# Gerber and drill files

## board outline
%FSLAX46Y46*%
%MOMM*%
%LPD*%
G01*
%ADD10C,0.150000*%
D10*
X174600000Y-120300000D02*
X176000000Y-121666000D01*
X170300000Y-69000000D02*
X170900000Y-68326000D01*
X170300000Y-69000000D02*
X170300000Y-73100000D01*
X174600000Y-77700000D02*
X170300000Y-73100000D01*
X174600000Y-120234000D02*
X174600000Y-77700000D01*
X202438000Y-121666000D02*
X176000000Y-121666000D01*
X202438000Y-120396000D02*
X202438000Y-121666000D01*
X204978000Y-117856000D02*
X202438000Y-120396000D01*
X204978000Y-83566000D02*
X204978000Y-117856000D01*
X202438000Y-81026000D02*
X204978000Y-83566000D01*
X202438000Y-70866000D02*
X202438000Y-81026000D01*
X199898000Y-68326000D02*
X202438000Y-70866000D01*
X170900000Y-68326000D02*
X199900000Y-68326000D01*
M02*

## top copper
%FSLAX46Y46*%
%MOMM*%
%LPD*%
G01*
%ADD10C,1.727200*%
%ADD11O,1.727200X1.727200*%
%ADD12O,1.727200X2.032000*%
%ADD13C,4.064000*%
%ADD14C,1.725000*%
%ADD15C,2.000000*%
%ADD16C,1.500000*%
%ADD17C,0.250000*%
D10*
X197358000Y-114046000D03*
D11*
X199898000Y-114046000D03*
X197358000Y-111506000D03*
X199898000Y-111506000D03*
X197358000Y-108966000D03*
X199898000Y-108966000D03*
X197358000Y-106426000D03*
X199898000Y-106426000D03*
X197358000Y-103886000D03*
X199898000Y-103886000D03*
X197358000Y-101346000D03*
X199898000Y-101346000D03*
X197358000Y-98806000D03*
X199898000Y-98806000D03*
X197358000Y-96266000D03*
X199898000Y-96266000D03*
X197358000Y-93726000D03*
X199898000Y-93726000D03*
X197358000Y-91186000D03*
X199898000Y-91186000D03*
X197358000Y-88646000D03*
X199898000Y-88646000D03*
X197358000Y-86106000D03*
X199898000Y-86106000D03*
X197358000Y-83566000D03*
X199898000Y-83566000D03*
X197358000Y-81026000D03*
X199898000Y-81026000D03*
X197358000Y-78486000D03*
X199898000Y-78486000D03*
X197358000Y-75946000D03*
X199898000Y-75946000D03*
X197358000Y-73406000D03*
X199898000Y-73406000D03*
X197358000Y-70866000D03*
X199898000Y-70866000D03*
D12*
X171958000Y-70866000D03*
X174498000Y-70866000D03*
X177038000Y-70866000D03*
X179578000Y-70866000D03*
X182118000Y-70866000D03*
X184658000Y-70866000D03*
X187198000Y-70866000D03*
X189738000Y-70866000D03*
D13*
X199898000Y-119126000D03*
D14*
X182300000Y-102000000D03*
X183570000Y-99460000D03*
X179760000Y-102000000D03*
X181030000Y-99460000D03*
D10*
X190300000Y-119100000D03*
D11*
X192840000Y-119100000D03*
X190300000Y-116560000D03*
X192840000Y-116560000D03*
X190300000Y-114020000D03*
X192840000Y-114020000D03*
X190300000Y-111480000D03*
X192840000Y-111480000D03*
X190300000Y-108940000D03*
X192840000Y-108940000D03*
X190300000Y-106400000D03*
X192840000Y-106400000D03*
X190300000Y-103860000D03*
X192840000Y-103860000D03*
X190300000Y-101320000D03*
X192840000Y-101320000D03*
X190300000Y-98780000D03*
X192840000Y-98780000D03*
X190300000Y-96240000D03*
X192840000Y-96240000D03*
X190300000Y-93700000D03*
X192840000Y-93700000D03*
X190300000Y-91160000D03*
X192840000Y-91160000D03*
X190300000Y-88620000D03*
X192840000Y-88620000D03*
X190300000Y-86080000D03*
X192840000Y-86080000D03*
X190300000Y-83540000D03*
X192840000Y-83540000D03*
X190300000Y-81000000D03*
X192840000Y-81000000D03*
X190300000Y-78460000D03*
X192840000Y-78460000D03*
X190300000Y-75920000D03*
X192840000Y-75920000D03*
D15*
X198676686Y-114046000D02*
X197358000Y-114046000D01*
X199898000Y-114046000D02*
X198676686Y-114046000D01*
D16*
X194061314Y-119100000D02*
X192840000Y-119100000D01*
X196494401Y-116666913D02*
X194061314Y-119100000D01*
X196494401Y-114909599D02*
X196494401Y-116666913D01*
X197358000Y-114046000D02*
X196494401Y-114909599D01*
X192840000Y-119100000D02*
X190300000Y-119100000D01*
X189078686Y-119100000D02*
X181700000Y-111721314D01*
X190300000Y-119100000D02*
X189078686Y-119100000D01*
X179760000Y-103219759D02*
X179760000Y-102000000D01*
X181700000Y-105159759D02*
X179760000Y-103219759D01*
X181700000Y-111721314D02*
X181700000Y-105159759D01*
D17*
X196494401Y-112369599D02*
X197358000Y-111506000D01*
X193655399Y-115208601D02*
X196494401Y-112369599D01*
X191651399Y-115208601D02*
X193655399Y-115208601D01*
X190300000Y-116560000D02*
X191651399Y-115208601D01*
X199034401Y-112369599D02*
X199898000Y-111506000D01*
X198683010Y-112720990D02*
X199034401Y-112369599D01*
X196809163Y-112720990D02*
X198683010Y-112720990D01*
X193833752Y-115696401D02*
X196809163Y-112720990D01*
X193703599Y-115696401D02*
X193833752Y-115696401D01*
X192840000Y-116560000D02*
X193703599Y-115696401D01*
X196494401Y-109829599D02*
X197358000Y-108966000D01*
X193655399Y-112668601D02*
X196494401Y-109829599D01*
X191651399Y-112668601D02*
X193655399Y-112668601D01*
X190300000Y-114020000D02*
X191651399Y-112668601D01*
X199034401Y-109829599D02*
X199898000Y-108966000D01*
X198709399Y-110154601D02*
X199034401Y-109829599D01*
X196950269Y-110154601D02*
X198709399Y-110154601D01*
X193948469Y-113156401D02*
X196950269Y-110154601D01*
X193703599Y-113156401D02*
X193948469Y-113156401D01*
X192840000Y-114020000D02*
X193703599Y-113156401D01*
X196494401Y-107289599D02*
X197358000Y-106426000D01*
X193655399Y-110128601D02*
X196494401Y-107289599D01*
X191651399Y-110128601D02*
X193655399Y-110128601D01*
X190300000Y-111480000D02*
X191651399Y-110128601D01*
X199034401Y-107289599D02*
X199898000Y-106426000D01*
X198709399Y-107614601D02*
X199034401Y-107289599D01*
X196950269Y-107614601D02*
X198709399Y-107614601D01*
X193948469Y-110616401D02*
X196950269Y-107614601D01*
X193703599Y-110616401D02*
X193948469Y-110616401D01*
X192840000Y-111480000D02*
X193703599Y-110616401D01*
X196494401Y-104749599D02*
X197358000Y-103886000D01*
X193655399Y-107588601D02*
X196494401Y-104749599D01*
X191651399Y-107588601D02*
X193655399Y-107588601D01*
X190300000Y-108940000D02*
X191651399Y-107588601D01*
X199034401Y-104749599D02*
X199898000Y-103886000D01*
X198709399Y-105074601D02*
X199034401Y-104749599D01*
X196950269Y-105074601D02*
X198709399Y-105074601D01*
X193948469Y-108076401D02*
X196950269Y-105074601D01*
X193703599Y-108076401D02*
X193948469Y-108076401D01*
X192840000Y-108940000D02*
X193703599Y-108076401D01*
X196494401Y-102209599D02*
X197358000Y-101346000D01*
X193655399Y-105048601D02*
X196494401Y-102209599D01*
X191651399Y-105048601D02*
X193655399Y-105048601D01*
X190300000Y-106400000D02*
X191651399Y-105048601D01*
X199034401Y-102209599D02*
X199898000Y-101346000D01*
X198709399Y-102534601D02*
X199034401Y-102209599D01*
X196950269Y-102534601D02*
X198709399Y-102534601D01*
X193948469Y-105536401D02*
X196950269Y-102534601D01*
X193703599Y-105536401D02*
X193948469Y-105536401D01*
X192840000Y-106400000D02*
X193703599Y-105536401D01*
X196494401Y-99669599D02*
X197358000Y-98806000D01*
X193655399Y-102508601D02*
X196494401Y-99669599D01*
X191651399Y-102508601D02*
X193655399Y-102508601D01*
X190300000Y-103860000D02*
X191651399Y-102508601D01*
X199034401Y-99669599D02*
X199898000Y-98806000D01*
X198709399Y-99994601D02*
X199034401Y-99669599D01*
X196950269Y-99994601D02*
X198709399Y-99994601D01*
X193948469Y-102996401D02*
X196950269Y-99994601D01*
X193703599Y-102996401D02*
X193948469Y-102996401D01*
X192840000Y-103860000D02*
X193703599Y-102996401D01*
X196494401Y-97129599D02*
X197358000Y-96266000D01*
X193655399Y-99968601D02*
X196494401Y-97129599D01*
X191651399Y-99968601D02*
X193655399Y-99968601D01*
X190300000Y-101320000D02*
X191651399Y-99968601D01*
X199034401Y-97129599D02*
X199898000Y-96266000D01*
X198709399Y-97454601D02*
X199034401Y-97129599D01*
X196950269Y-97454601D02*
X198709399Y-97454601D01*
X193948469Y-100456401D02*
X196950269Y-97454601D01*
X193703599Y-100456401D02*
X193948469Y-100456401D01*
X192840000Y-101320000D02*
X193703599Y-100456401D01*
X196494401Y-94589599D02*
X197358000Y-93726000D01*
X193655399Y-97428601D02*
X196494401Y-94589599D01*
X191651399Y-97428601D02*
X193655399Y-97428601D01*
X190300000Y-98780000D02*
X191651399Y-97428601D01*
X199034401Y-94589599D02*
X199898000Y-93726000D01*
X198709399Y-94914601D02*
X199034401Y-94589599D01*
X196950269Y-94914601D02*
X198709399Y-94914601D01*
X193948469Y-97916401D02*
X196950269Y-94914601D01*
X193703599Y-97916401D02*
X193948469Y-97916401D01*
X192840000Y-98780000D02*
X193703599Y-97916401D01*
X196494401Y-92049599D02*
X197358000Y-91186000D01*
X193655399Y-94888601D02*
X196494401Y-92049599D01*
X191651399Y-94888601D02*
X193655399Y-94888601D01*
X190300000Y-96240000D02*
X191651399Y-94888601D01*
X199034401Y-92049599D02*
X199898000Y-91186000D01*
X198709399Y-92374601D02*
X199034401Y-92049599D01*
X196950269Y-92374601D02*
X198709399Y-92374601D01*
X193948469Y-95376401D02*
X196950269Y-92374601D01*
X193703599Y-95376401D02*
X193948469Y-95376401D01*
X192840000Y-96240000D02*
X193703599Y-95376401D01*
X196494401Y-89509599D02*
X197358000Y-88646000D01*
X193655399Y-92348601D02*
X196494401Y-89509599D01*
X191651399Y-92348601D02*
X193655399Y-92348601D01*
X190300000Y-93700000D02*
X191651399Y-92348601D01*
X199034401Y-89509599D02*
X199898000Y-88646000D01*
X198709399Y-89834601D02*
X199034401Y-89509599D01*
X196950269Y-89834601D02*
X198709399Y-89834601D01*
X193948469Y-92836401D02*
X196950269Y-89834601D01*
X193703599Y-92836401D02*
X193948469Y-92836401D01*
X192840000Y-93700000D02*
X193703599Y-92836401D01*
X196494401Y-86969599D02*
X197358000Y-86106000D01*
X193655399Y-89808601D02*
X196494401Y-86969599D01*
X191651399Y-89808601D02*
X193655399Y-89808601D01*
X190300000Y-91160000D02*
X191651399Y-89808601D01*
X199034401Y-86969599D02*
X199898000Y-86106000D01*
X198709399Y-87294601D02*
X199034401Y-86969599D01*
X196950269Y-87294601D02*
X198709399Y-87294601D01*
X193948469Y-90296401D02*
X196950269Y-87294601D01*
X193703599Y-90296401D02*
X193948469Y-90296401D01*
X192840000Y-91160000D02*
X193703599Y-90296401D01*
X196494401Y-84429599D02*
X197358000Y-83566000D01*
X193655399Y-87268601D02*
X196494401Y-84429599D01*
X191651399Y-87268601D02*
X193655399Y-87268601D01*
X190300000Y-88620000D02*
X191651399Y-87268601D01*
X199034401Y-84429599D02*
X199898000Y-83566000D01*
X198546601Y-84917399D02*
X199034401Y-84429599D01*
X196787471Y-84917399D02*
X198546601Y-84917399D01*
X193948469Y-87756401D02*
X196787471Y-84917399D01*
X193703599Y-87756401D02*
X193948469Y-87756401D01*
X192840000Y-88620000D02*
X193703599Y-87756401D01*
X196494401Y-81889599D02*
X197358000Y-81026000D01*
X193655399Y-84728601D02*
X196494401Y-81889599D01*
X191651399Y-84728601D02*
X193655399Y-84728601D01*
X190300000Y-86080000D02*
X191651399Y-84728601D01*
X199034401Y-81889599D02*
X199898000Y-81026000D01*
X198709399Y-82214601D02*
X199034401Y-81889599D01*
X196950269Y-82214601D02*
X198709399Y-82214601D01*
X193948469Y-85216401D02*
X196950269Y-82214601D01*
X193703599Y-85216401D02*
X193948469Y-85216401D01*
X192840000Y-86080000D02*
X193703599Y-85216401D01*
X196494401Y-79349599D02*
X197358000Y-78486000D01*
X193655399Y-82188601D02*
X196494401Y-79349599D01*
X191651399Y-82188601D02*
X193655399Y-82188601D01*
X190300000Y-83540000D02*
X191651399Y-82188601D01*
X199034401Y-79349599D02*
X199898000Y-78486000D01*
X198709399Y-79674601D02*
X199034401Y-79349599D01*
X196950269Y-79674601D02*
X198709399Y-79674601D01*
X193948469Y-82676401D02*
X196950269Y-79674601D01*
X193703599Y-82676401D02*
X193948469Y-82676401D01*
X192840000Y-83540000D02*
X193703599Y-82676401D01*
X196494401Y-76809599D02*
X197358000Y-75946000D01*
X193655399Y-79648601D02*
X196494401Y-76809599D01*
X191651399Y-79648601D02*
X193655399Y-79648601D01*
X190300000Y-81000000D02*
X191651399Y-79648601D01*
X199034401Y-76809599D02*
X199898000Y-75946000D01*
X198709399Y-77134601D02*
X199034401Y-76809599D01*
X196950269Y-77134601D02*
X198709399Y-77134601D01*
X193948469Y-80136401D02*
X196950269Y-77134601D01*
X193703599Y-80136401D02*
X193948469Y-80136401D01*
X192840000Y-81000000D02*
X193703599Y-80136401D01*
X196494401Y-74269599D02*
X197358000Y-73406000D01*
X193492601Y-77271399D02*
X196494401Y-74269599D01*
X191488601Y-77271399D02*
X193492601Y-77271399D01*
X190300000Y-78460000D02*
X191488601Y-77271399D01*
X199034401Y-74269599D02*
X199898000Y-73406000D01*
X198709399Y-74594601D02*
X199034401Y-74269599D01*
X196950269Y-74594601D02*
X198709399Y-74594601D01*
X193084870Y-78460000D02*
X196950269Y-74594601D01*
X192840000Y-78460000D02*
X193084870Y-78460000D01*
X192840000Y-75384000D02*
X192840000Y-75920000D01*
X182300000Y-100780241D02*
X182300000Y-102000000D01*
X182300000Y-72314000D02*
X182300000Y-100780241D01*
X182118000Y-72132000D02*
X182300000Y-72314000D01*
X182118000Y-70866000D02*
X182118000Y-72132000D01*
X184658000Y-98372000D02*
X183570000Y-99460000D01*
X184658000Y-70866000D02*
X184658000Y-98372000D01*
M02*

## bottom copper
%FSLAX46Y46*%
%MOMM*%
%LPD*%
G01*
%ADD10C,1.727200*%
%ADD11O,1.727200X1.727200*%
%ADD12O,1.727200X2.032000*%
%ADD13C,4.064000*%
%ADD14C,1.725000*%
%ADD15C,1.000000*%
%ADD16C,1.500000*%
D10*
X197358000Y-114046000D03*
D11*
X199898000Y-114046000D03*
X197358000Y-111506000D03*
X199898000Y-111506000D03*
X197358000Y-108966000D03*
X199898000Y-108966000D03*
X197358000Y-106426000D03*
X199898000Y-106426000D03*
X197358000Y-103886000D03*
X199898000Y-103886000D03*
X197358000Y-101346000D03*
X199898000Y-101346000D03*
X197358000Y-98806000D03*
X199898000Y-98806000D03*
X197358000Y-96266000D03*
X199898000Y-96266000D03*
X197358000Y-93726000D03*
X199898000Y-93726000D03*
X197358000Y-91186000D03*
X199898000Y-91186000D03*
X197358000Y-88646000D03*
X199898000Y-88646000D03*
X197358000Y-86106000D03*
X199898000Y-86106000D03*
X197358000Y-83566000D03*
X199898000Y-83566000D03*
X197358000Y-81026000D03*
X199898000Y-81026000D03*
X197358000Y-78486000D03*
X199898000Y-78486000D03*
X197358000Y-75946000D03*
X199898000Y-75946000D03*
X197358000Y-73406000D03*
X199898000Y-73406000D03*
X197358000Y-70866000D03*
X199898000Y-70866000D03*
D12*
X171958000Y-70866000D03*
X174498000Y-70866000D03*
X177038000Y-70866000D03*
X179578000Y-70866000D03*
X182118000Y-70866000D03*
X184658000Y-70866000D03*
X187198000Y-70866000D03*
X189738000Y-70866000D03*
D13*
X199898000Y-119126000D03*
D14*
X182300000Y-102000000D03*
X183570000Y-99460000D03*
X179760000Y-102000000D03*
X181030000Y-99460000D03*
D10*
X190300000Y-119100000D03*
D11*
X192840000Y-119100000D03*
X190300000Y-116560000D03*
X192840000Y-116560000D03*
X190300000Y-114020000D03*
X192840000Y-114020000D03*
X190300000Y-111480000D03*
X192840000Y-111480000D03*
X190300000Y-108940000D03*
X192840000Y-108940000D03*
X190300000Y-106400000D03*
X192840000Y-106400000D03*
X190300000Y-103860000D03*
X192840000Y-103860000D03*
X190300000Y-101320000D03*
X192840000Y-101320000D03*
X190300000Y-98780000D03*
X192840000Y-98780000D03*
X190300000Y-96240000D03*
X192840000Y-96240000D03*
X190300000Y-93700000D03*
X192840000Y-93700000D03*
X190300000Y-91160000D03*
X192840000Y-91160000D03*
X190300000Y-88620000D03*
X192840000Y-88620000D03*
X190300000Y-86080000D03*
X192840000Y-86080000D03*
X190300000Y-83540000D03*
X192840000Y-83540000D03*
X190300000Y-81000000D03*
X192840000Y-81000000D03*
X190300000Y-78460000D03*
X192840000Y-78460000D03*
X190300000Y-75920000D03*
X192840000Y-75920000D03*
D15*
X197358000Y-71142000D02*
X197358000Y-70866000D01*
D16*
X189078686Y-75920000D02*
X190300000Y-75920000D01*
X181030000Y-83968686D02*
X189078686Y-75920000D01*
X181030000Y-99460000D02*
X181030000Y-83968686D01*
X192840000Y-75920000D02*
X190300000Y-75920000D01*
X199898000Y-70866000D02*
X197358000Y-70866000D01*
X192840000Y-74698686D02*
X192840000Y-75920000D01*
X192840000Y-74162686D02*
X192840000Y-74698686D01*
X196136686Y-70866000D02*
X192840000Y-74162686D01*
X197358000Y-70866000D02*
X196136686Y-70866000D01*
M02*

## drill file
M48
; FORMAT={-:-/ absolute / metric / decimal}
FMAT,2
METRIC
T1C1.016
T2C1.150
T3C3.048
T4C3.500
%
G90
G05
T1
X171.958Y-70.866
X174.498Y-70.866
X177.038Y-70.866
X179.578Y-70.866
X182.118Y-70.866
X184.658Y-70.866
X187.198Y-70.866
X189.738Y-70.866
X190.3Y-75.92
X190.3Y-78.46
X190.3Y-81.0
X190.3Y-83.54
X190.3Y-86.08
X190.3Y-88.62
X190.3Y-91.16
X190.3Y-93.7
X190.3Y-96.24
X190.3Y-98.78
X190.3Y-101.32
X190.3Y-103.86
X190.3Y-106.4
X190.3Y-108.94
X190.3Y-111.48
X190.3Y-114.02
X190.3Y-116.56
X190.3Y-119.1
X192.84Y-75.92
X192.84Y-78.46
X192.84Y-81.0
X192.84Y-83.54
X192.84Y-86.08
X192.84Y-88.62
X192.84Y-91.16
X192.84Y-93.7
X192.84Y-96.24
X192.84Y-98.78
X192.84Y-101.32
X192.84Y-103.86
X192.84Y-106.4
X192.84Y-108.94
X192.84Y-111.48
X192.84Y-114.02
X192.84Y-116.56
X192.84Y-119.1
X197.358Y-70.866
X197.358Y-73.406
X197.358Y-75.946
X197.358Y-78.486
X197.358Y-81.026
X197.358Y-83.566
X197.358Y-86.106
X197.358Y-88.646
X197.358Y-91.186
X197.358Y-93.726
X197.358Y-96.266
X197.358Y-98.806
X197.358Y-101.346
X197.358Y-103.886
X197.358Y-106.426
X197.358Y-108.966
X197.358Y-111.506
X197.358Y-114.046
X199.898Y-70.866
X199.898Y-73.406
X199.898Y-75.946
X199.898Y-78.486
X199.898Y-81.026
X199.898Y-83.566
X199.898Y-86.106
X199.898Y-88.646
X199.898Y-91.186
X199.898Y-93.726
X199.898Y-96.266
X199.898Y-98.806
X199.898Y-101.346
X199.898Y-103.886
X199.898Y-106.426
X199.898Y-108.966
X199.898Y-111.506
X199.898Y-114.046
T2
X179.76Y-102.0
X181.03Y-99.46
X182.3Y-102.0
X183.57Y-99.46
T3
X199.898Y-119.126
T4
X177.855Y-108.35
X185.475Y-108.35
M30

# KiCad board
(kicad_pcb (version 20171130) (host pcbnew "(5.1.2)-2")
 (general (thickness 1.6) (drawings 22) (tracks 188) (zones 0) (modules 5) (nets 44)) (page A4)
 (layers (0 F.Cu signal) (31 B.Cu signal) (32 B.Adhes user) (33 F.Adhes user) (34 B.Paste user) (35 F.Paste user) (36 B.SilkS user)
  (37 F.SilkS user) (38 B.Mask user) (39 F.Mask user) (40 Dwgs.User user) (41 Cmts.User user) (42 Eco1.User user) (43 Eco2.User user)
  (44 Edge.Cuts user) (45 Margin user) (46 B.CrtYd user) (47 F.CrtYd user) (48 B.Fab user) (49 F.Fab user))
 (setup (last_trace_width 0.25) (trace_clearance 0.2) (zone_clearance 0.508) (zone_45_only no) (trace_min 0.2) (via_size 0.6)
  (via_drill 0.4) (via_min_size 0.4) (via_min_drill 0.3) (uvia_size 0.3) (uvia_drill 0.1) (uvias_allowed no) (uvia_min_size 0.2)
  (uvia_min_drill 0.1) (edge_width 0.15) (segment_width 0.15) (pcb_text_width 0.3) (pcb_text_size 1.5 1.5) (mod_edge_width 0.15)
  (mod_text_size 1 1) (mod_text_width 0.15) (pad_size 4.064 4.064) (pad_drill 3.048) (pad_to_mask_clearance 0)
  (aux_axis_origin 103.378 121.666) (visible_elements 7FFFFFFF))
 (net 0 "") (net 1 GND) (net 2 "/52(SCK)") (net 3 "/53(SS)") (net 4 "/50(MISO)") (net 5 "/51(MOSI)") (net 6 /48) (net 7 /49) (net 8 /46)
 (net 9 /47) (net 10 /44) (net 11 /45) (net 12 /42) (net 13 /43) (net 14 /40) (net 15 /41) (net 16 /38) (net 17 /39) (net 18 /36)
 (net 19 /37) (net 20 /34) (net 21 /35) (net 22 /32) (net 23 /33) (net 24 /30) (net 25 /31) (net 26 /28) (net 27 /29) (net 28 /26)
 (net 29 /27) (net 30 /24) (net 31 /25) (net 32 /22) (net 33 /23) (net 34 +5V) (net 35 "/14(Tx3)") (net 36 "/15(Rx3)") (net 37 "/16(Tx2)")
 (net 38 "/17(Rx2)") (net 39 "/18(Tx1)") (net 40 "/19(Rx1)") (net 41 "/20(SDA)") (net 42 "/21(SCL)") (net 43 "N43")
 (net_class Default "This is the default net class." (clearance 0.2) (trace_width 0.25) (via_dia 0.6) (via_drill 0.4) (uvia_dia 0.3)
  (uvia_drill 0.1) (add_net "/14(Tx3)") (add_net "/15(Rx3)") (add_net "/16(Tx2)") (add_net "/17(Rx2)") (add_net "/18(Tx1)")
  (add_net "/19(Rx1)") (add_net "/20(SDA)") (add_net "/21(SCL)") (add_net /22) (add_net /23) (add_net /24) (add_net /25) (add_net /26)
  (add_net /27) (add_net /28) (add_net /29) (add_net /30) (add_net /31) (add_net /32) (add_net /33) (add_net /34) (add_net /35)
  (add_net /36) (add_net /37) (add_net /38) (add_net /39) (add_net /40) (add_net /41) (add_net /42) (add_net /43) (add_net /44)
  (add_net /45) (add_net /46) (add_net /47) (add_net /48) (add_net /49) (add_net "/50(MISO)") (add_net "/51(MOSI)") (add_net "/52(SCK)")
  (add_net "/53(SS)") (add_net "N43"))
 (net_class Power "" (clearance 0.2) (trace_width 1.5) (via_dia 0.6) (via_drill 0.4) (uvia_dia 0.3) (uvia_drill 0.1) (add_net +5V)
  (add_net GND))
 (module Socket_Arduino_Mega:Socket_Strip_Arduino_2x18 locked (layer F.Cu) (at 197.358 114.046 90)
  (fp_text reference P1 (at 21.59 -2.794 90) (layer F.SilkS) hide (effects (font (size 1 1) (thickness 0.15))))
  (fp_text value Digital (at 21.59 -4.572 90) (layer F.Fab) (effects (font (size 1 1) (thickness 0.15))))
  (pad 1 thru_hole circle (at 0 0 90) (size 1.7272 1.7272) (drill 1.016) (layers *.Cu *.Mask F.SilkS) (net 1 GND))
  (pad 2 thru_hole oval (at 0 2.54 90) (size 1.7272 1.7272) (drill 1.016) (layers *.Cu *.Mask F.SilkS) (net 1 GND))
  (pad 3 thru_hole oval (at 2.54 0 90) (size 1.7272 1.7272) (drill 1.016) (layers *.Cu *.Mask F.SilkS) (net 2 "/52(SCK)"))
  (pad 4 thru_hole oval (at 2.54 2.54 90) (size 1.7272 1.7272) (drill 1.016) (layers *.Cu *.Mask F.SilkS) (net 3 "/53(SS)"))
  (pad 5 thru_hole oval (at 5.08 0 90) (size 1.7272 1.7272) (drill 1.016) (layers *.Cu *.Mask F.SilkS) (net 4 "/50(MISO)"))
  (pad 6 thru_hole oval (at 5.08 2.54 90) (size 1.7272 1.7272) (drill 1.016) (layers *.Cu *.Mask F.SilkS) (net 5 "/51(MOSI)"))
  (pad 7 thru_hole oval (at 7.62 0 90) (size 1.7272 1.7272) (drill 1.016) (layers *.Cu *.Mask F.SilkS) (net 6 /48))
  (pad 8 thru_hole oval (at 7.62 2.54 90) (size 1.7272 1.7272) (drill 1.016) (layers *.Cu *.Mask F.SilkS) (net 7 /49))
  (pad 9 thru_hole oval (at 10.16 0 90) (size 1.7272 1.7272) (drill 1.016) (layers *.Cu *.Mask F.SilkS) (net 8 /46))
  (pad 10 thru_hole oval (at 10.16 2.54 90) (size 1.7272 1.7272) (drill 1.016) (layers *.Cu *.Mask F.SilkS) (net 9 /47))
  (pad 11 thru_hole oval (at 12.7 0 90) (size 1.7272 1.7272) (drill 1.016) (layers *.Cu *.Mask F.SilkS) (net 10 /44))
  (pad 12 thru_hole oval (at 12.7 2.54 90) (size 1.7272 1.7272) (drill 1.016) (layers *.Cu *.Mask F.SilkS) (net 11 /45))
  (pad 13 thru_hole oval (at 15.24 0 90) (size 1.7272 1.7272) (drill 1.016) (layers *.Cu *.Mask F.SilkS) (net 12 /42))
  (pad 14 thru_hole oval (at 15.24 2.54 90) (size 1.7272 1.7272) (drill 1.016) (layers *.Cu *.Mask F.SilkS) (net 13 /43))
  (pad 15 thru_hole oval (at 17.78 0 90) (size 1.7272 1.7272) (drill 1.016) (layers *.Cu *.Mask F.SilkS) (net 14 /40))
  (pad 16 thru_hole oval (at 17.78 2.54 90) (size 1.7272 1.7272) (drill 1.016) (layers *.Cu *.Mask F.SilkS) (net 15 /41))
  (pad 17 thru_hole oval (at 20.32 0 90) (size 1.7272 1.7272) (drill 1.016) (layers *.Cu *.Mask F.SilkS) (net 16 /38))
  (pad 18 thru_hole oval (at 20.32 2.54 90) (size 1.7272 1.7272) (drill 1.016) (layers *.Cu *.Mask F.SilkS) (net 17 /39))
  (pad 19 thru_hole oval (at 22.86 0 90) (size 1.7272 1.7272) (drill 1.016) (layers *.Cu *.Mask F.SilkS) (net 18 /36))
  (pad 20 thru_hole oval (at 22.86 2.54 90) (size 1.7272 1.7272) (drill 1.016) (layers *.Cu *.Mask F.SilkS) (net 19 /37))
  (pad 21 thru_hole oval (at 25.4 0 90) (size 1.7272 1.7272) (drill 1.016) (layers *.Cu *.Mask F.SilkS) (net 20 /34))
  (pad 22 thru_hole oval (at 25.4 2.54 90) (size 1.7272 1.7272) (drill 1.016) (layers *.Cu *.Mask F.SilkS) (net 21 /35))
  (pad 23 thru_hole oval (at 27.94 0 90) (size 1.7272 1.7272) (drill 1.016) (layers *.Cu *.Mask F.SilkS) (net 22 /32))
  (pad 24 thru_hole oval (at 27.94 2.54 90) (size 1.7272 1.7272) (drill 1.016) (layers *.Cu *.Mask F.SilkS) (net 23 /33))
  (pad 25 thru_hole oval (at 30.48 0 90) (size 1.7272 1.7272) (drill 1.016) (layers *.Cu *.Mask F.SilkS) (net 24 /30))
  (pad 26 thru_hole oval (at 30.48 2.54 90) (size 1.7272 1.7272) (drill 1.016) (layers *.Cu *.Mask F.SilkS) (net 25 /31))
  (pad 27 thru_hole oval (at 33.02 0 90) (size 1.7272 1.7272) (drill 1.016) (layers *.Cu *.Mask F.SilkS) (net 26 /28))
  (pad 28 thru_hole oval (at 33.02 2.54 90) (size 1.7272 1.7272) (drill 1.016) (layers *.Cu *.Mask F.SilkS) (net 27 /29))
  (pad 29 thru_hole oval (at 35.56 0 90) (size 1.7272 1.7272) (drill 1.016) (layers *.Cu *.Mask F.SilkS) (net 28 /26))
  (pad 30 thru_hole oval (at 35.56 2.54 90) (size 1.7272 1.7272) (drill 1.016) (layers *.Cu *.Mask F.SilkS) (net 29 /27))
  (pad 31 thru_hole oval (at 38.1 0 90) (size 1.7272 1.7272) (drill 1.016) (layers *.Cu *.Mask F.SilkS) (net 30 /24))
  (pad 32 thru_hole oval (at 38.1 2.54 90) (size 1.7272 1.7272) (drill 1.016) (layers *.Cu *.Mask F.SilkS) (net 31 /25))
  (pad 33 thru_hole oval (at 40.64 0 90) (size 1.7272 1.7272) (drill 1.016) (layers *.Cu *.Mask F.SilkS) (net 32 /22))
  (pad 34 thru_hole oval (at 40.64 2.54 90) (size 1.7272 1.7272) (drill 1.016) (layers *.Cu *.Mask F.SilkS) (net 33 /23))
  (pad 35 thru_hole oval (at 43.18 0 90) (size 1.7272 1.7272) (drill 1.016) (layers *.Cu *.Mask F.SilkS) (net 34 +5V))
  (pad 36 thru_hole oval (at 43.18 2.54 90) (size 1.7272 1.7272) (drill 1.016) (layers *.Cu *.Mask F.SilkS) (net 34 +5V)))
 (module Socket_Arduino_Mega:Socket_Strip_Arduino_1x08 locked (layer F.Cu) (at 171.958 70.866)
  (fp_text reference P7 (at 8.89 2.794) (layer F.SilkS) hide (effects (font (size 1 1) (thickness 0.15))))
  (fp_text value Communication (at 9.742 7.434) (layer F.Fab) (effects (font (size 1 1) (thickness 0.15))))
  (pad 1 thru_hole oval (at 0 0) (size 1.7272 2.032) (drill 1.016) (layers *.Cu *.Mask F.SilkS) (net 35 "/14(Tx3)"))
  (pad 2 thru_hole oval (at 2.54 0) (size 1.7272 2.032) (drill 1.016) (layers *.Cu *.Mask F.SilkS) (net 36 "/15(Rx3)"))
  (pad 3 thru_hole oval (at 5.08 0) (size 1.7272 2.032) (drill 1.016) (layers *.Cu *.Mask F.SilkS) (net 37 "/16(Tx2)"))
  (pad 4 thru_hole oval (at 7.62 0) (size 1.7272 2.032) (drill 1.016) (layers *.Cu *.Mask F.SilkS) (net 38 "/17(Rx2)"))
  (pad 5 thru_hole oval (at 10.16 0) (size 1.7272 2.032) (drill 1.016) (layers *.Cu *.Mask F.SilkS) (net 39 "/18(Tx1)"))
  (pad 6 thru_hole oval (at 12.7 0) (size 1.7272 2.032) (drill 1.016) (layers *.Cu *.Mask F.SilkS) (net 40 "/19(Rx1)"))
  (pad 7 thru_hole oval (at 15.24 0) (size 1.7272 2.032) (drill 1.016) (layers *.Cu *.Mask F.SilkS) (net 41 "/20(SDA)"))
  (pad 8 thru_hole oval (at 17.78 0) (size 1.7272 2.032) (drill 1.016) (layers *.Cu *.Mask F.SilkS) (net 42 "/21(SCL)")))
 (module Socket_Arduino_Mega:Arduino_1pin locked (layer F.Cu) (at 199.898 119.126)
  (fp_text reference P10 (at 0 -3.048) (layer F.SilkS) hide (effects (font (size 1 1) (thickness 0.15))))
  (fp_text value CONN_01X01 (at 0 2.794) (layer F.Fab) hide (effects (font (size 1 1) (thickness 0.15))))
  (pad 1 thru_hole circle (at 0 0) (size 4.064 4.064) (drill 3.048) (layers *.Cu *.Mask F.SilkS) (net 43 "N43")))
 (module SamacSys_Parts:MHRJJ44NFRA (layer F.Cu) (at 182.3 102)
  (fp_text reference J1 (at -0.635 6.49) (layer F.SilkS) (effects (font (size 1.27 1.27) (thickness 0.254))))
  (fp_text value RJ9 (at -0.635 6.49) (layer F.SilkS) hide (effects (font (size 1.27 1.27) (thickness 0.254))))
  (pad 1 thru_hole circle (at 0 0) (size 1.725 1.725) (drill 1.15) (layers *.Cu *.Mask) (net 39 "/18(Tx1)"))
  (pad 2 thru_hole circle (at 1.27 -2.54) (size 1.725 1.725) (drill 1.15) (layers *.Cu *.Mask) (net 40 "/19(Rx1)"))
  (pad 3 thru_hole circle (at -2.54 0) (size 1.725 1.725) (drill 1.15) (layers *.Cu *.Mask) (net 1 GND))
  (pad 4 thru_hole circle (at -1.27 -2.54) (size 1.725 1.725) (drill 1.15) (layers *.Cu *.Mask) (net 34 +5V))
  (pad MH1 np_thru_hole circle (at 3.175 6.35) (size 3.5 0) (drill 3.5) (layers *.Cu *.Mask))
  (pad MH2 np_thru_hole circle (at -4.445 6.35) (size 3.5 0) (drill 3.5) (layers *.Cu *.Mask)))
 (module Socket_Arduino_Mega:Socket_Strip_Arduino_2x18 (layer F.Cu) (at 190.3 119.1 90)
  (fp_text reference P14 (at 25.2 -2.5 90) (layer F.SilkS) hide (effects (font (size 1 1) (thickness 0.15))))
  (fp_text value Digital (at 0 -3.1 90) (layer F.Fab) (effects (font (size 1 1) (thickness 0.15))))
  (pad 1 thru_hole circle (at 0 0 90) (size 1.7272 1.7272) (drill 1.016) (layers *.Cu *.Mask F.SilkS) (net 1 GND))
  (pad 2 thru_hole oval (at 0 2.54 90) (size 1.7272 1.7272) (drill 1.016) (layers *.Cu *.Mask F.SilkS) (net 1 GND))
  (pad 3 thru_hole oval (at 2.54 0 90) (size 1.7272 1.7272) (drill 1.016) (layers *.Cu *.Mask F.SilkS) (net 2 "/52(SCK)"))
  (pad 4 thru_hole oval (at 2.54 2.54 90) (size 1.7272 1.7272) (drill 1.016) (layers *.Cu *.Mask F.SilkS) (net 3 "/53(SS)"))
  (pad 5 thru_hole oval (at 5.08 0 90) (size 1.7272 1.7272) (drill 1.016) (layers *.Cu *.Mask F.SilkS) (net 4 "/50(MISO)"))
  (pad 6 thru_hole oval (at 5.08 2.54 90) (size 1.7272 1.7272) (drill 1.016) (layers *.Cu *.Mask F.SilkS) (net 5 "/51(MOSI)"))
  (pad 7 thru_hole oval (at 7.62 0 90) (size 1.7272 1.7272) (drill 1.016) (layers *.Cu *.Mask F.SilkS) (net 6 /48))
  (pad 8 thru_hole oval (at 7.62 2.54 90) (size 1.7272 1.7272) (drill 1.016) (layers *.Cu *.Mask F.SilkS) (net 7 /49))
  (pad 9 thru_hole oval (at 10.16 0 90) (size 1.7272 1.7272) (drill 1.016) (layers *.Cu *.Mask F.SilkS) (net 8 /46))
  (pad 10 thru_hole oval (at 10.16 2.54 90) (size 1.7272 1.7272) (drill 1.016) (layers *.Cu *.Mask F.SilkS) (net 9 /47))
  (pad 11 thru_hole oval (at 12.7 0 90) (size 1.7272 1.7272) (drill 1.016) (layers *.Cu *.Mask F.SilkS) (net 10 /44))
  (pad 12 thru_hole oval (at 12.7 2.54 90) (size 1.7272 1.7272) (drill 1.016) (layers *.Cu *.Mask F.SilkS) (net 11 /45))
  (pad 13 thru_hole oval (at 15.24 0 90) (size 1.7272 1.7272) (drill 1.016) (layers *.Cu *.Mask F.SilkS) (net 12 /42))
  (pad 14 thru_hole oval (at 15.24 2.54 90) (size 1.7272 1.7272) (drill 1.016) (layers *.Cu *.Mask F.SilkS) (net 13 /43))
  (pad 15 thru_hole oval (at 17.78 0 90) (size 1.7272 1.7272) (drill 1.016) (layers *.Cu *.Mask F.SilkS) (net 14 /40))
  (pad 16 thru_hole oval (at 17.78 2.54 90) (size 1.7272 1.7272) (drill 1.016) (layers *.Cu *.Mask F.SilkS) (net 15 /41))
  (pad 17 thru_hole oval (at 20.32 0 90) (size 1.7272 1.7272) (drill 1.016) (layers *.Cu *.Mask F.SilkS) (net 16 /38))
  (pad 18 thru_hole oval (at 20.32 2.54 90) (size 1.7272 1.7272) (drill 1.016) (layers *.Cu *.Mask F.SilkS) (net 17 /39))
  (pad 19 thru_hole oval (at 22.86 0 90) (size 1.7272 1.7272) (drill 1.016) (layers *.Cu *.Mask F.SilkS) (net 18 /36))
  (pad 20 thru_hole oval (at 22.86 2.54 90) (size 1.7272 1.7272) (drill 1.016) (layers *.Cu *.Mask F.SilkS) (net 19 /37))
  (pad 21 thru_hole oval (at 25.4 0 90) (size 1.7272 1.7272) (drill 1.016) (layers *.Cu *.Mask F.SilkS) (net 20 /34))
  (pad 22 thru_hole oval (at 25.4 2.54 90) (size 1.7272 1.7272) (drill 1.016) (layers *.Cu *.Mask F.SilkS) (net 21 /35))
  (pad 23 thru_hole oval (at 27.94 0 90) (size 1.7272 1.7272) (drill 1.016) (layers *.Cu *.Mask F.SilkS) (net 22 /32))
  (pad 24 thru_hole oval (at 27.94 2.54 90) (size 1.7272 1.7272) (drill 1.016) (layers *.Cu *.Mask F.SilkS) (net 23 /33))
  (pad 25 thru_hole oval (at 30.48 0 90) (size 1.7272 1.7272) (drill 1.016) (layers *.Cu *.Mask F.SilkS) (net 24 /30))
  (pad 26 thru_hole oval (at 30.48 2.54 90) (size 1.7272 1.7272) (drill 1.016) (layers *.Cu *.Mask F.SilkS) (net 25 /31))
  (pad 27 thru_hole oval (at 33.02 0 90) (size 1.7272 1.7272) (drill 1.016) (layers *.Cu *.Mask F.SilkS) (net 26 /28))
  (pad 28 thru_hole oval (at 33.02 2.54 90) (size 1.7272 1.7272) (drill 1.016) (layers *.Cu *.Mask F.SilkS) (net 27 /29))
  (pad 29 thru_hole oval (at 35.56 0 90) (size 1.7272 1.7272) (drill 1.016) (layers *.Cu *.Mask F.SilkS) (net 28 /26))
  (pad 30 thru_hole oval (at 35.56 2.54 90) (size 1.7272 1.7272) (drill 1.016) (layers *.Cu *.Mask F.SilkS) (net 29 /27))
  (pad 31 thru_hole oval (at 38.1 0 90) (size 1.7272 1.7272) (drill 1.016) (layers *.Cu *.Mask F.SilkS) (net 30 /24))
  (pad 32 thru_hole oval (at 38.1 2.54 90) (size 1.7272 1.7272) (drill 1.016) (layers *.Cu *.Mask F.SilkS) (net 31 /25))
  (pad 33 thru_hole oval (at 40.64 0 90) (size 1.7272 1.7272) (drill 1.016) (layers *.Cu *.Mask F.SilkS) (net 32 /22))
  (pad 34 thru_hole oval (at 40.64 2.54 90) (size 1.7272 1.7272) (drill 1.016) (layers *.Cu *.Mask F.SilkS) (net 33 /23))
  (pad 35 thru_hole oval (at 43.18 0 90) (size 1.7272 1.7272) (drill 1.016) (layers *.Cu *.Mask F.SilkS) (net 34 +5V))
  (pad 36 thru_hole oval (at 43.18 2.54 90) (size 1.7272 1.7272) (drill 1.016) (layers *.Cu *.Mask F.SilkS) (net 34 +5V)))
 (gr_line (start 174.6 120.3) (end 176 121.666) (layer Edge.Cuts) (width 0.15))
 (gr_line (start 170.3 69) (end 170.9 68.326) (layer Edge.Cuts) (width 0.15))
 (gr_line (start 170.3 69) (end 170.3 73.1) (layer Edge.Cuts) (width 0.15))
 (gr_line (start 174.6 77.7) (end 170.3 73.1) (layer Edge.Cuts) (width 0.15))
 (gr_line (start 174.6 120.234) (end 174.6 77.7) (layer Edge.Cuts) (width 0.15))
 (gr_line (start 202.438 121.666) (end 176 121.666) (angle 90) (layer Edge.Cuts) (width 0.15))
 (gr_line (start 202.438 120.396) (end 202.438 121.666) (angle 90) (layer Edge.Cuts) (width 0.15))
 (gr_line (start 204.978 117.856) (end 202.438 120.396) (angle 90) (layer Edge.Cuts) (width 0.15))
 (gr_line (start 204.978 83.566) (end 204.978 117.856) (angle 90) (layer Edge.Cuts) (width 0.15))
 (gr_line (start 202.438 81.026) (end 204.978 83.566) (angle 90) (layer Edge.Cuts) (width 0.15))
 (gr_line (start 202.438 70.866) (end 202.438 81.026) (angle 90) (layer Edge.Cuts) (width 0.15))
 (gr_line (start 199.898 68.326) (end 202.438 70.866) (angle 90) (layer Edge.Cuts) (width 0.15))
 (gr_line (start 170.9 68.326) (end 199.9 68.326) (angle 90) (layer Edge.Cuts) (width 0.15))
 (segment (start 198.676686 114.046) (end 197.358 114.046) (width 2) (layer F.Cu) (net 1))
 (segment (start 199.898 114.046) (end 198.676686 114.046) (width 2) (layer F.Cu) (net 1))
 (segment (start 194.061314 119.1) (end 192.84 119.1) (width 1.5) (layer F.Cu) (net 1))
 (segment (start 196.494401 116.666913) (end 194.061314 119.1) (width 1.5) (layer F.Cu) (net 1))
 (segment (start 196.494401 114.909599) (end 196.494401 116.666913) (width 1.5) (layer F.Cu) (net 1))
 (segment (start 197.358 114.046) (end 196.494401 114.909599) (width 1.5) (layer F.Cu) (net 1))
 (segment (start 192.84 119.1) (end 190.3 119.1) (width 1.5) (layer F.Cu) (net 1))
 (segment (start 189.078686 119.1) (end 181.7 111.721314) (width 1.5) (layer F.Cu) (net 1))
 (segment (start 190.3 119.1) (end 189.078686 119.1) (width 1.5) (layer F.Cu) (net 1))
 (segment (start 179.76 103.219759) (end 179.76 102) (width 1.5) (layer F.Cu) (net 1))
 (segment (start 181.7 105.159759) (end 179.76 103.219759) (width 1.5) (layer F.Cu) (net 1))
 (segment (start 181.7 111.721314) (end 181.7 105.159759) (width 1.5) (layer F.Cu) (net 1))
 (segment (start 196.494401 112.369599) (end 197.358 111.506) (width 0.25) (layer F.Cu) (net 2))
 (segment (start 193.655399 115.208601) (end 196.494401 112.369599) (width 0.25) (layer F.Cu) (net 2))
 (segment (start 191.651399 115.208601) (end 193.655399 115.208601) (width 0.25) (layer F.Cu) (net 2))
 (segment (start 190.3 116.56) (end 191.651399 115.208601) (width 0.25) (layer F.Cu) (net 2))
 (segment (start 199.034401 112.369599) (end 199.898 111.506) (width 0.25) (layer F.Cu) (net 3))
 (segment (start 198.68301 112.72099) (end 199.034401 112.369599) (width 0.25) (layer F.Cu) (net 3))
 (segment (start 196.809163 112.72099) (end 198.68301 112.72099) (width 0.25) (layer F.Cu) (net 3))
 (segment (start 193.833752 115.696401) (end 196.809163 112.72099) (width 0.25) (layer F.Cu) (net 3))
 (segment (start 193.703599 115.696401) (end 193.833752 115.696401) (width 0.25) (layer F.Cu) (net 3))
 (segment (start 192.84 116.56) (end 193.703599 115.696401) (width 0.25) (layer F.Cu) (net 3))
 (segment (start 196.494401 109.829599) (end 197.358 108.966) (width 0.25) (layer F.Cu) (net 4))
 (segment (start 193.655399 112.668601) (end 196.494401 109.829599) (width 0.25) (layer F.Cu) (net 4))
 (segment (start 191.651399 112.668601) (end 193.655399 112.668601) (width 0.25) (layer F.Cu) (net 4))
 (segment (start 190.3 114.02) (end 191.651399 112.668601) (width 0.25) (layer F.Cu) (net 4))
 (segment (start 199.034401 109.829599) (end 199.898 108.966) (width 0.25) (layer F.Cu) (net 5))
 (segment (start 198.709399 110.154601) (end 199.034401 109.829599) (width 0.25) (layer F.Cu) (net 5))
 (segment (start 196.950269 110.154601) (end 198.709399 110.154601) (width 0.25) (layer F.Cu) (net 5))
 (segment (start 193.948469 113.156401) (end 196.950269 110.154601) (width 0.25) (layer F.Cu) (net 5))
 (segment (start 193.703599 113.156401) (end 193.948469 113.156401) (width 0.25) (layer F.Cu) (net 5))
 (segment (start 192.84 114.02) (end 193.703599 113.156401) (width 0.25) (layer F.Cu) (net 5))
 (segment (start 196.494401 107.289599) (end 197.358 106.426) (width 0.25) (layer F.Cu) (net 6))
 (segment (start 193.655399 110.128601) (end 196.494401 107.289599) (width 0.25) (layer F.Cu) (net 6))
 (segment (start 191.651399 110.128601) (end 193.655399 110.128601) (width 0.25) (layer F.Cu) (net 6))
 (segment (start 190.3 111.48) (end 191.651399 110.128601) (width 0.25) (layer F.Cu) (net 6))
 (segment (start 199.034401 107.289599) (end 199.898 106.426) (width 0.25) (layer F.Cu) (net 7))
 (segment (start 198.709399 107.614601) (end 199.034401 107.289599) (width 0.25) (layer F.Cu) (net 7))
 (segment (start 196.950269 107.614601) (end 198.709399 107.614601) (width 0.25) (layer F.Cu) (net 7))
 (segment (start 193.948469 110.616401) (end 196.950269 107.614601) (width 0.25) (layer F.Cu) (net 7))
 (segment (start 193.703599 110.616401) (end 193.948469 110.616401) (width 0.25) (layer F.Cu) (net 7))
 (segment (start 192.84 111.48) (end 193.703599 110.616401) (width 0.25) (layer F.Cu) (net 7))
 (segment (start 196.494401 104.749599) (end 197.358 103.886) (width 0.25) (layer F.Cu) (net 8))
 (segment (start 193.655399 107.588601) (end 196.494401 104.749599) (width 0.25) (layer F.Cu) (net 8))
 (segment (start 191.651399 107.588601) (end 193.655399 107.588601) (width 0.25) (layer F.Cu) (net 8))
 (segment (start 190.3 108.94) (end 191.651399 107.588601) (width 0.25) (layer F.Cu) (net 8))
 (segment (start 199.034401 104.749599) (end 199.898 103.886) (width 0.25) (layer F.Cu) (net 9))
 (segment (start 198.709399 105.074601) (end 199.034401 104.749599) (width 0.25) (layer F.Cu) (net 9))
 (segment (start 196.950269 105.074601) (end 198.709399 105.074601) (width 0.25) (layer F.Cu) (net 9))
 (segment (start 193.948469 108.076401) (end 196.950269 105.074601) (width 0.25) (layer F.Cu) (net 9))
 (segment (start 193.703599 108.076401) (end 193.948469 108.076401) (width 0.25) (layer F.Cu) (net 9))
 (segment (start 192.84 108.94) (end 193.703599 108.076401) (width 0.25) (layer F.Cu) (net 9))
 (segment (start 196.494401 102.209599) (end 197.358 101.346) (width 0.25) (layer F.Cu) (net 10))
 (segment (start 193.655399 105.048601) (end 196.494401 102.209599) (width 0.25) (layer F.Cu) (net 10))
 (segment (start 191.651399 105.048601) (end 193.655399 105.048601) (width 0.25) (layer F.Cu) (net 10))
 (segment (start 190.3 106.4) (end 191.651399 105.048601) (width 0.25) (layer F.Cu) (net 10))
 (segment (start 199.034401 102.209599) (end 199.898 101.346) (width 0.25) (layer F.Cu) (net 11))
 (segment (start 198.709399 102.534601) (end 199.034401 102.209599) (width 0.25) (layer F.Cu) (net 11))
 (segment (start 196.950269 102.534601) (end 198.709399 102.534601) (width 0.25) (layer F.Cu) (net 11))
 (segment (start 193.948469 105.536401) (end 196.950269 102.534601) (width 0.25) (layer F.Cu) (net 11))
 (segment (start 193.703599 105.536401) (end 193.948469 105.536401) (width 0.25) (layer F.Cu) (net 11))
 (segment (start 192.84 106.4) (end 193.703599 105.536401) (width 0.25) (layer F.Cu) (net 11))
 (segment (start 196.494401 99.669599) (end 197.358 98.806) (width 0.25) (layer F.Cu) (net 12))
 (segment (start 193.655399 102.508601) (end 196.494401 99.669599) (width 0.25) (layer F.Cu) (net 12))
 (segment (start 191.651399 102.508601) (end 193.655399 102.508601) (width 0.25) (layer F.Cu) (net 12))
 (segment (start 190.3 103.86) (end 191.651399 102.508601) (width 0.25) (layer F.Cu) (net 12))
 (segment (start 199.034401 99.669599) (end 199.898 98.806) (width 0.25) (layer F.Cu) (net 13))
 (segment (start 198.709399 99.994601) (end 199.034401 99.669599) (width 0.25) (layer F.Cu) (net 13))
 (segment (start 196.950269 99.994601) (end 198.709399 99.994601) (width 0.25) (layer F.Cu) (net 13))
 (segment (start 193.948469 102.996401) (end 196.950269 99.994601) (width 0.25) (layer F.Cu) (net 13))
 (segment (start 193.703599 102.996401) (end 193.948469 102.996401) (width 0.25) (layer F.Cu) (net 13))
 (segment (start 192.84 103.86) (end 193.703599 102.996401) (width 0.25) (layer F.Cu) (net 13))
 (segment (start 196.494401 97.129599) (end 197.358 96.266) (width 0.25) (layer F.Cu) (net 14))
 (segment (start 193.655399 99.968601) (end 196.494401 97.129599) (width 0.25) (layer F.Cu) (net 14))
 (segment (start 191.651399 99.968601) (end 193.655399 99.968601) (width 0.25) (layer F.Cu) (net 14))
 (segment (start 190.3 101.32) (end 191.651399 99.968601) (width 0.25) (layer F.Cu) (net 14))
 (segment (start 199.034401 97.129599) (end 199.898 96.266) (width 0.25) (layer F.Cu) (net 15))
 (segment (start 198.709399 97.454601) (end 199.034401 97.129599) (width 0.25) (layer F.Cu) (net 15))
 (segment (start 196.950269 97.454601) (end 198.709399 97.454601) (width 0.25) (layer F.Cu) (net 15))
 (segment (start 193.948469 100.456401) (end 196.950269 97.454601) (width 0.25) (layer F.Cu) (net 15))
 (segment (start 193.703599 100.456401) (end 193.948469 100.456401) (width 0.25) (layer F.Cu) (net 15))
 (segment (start 192.84 101.32) (end 193.703599 100.456401) (width 0.25) (layer F.Cu) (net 15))
 (segment (start 196.494401 94.589599) (end 197.358 93.726) (width 0.25) (layer F.Cu) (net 16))
 (segment (start 193.655399 97.428601) (end 196.494401 94.589599) (width 0.25) (layer F.Cu) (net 16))
 (segment (start 191.651399 97.428601) (end 193.655399 97.428601) (width 0.25) (layer F.Cu) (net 16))
 (segment (start 190.3 98.78) (end 191.651399 97.428601) (width 0.25) (layer F.Cu) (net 16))
 (segment (start 199.034401 94.589599) (end 199.898 93.726) (width 0.25) (layer F.Cu) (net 17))
 (segment (start 198.709399 94.914601) (end 199.034401 94.589599) (width 0.25) (layer F.Cu) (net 17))
 (segment (start 196.950269 94.914601) (end 198.709399 94.914601) (width 0.25) (layer F.Cu) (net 17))
 (segment (start 193.948469 97.916401) (end 196.950269 94.914601) (width 0.25) (layer F.Cu) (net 17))
 (segment (start 193.703599 97.916401) (end 193.948469 97.916401) (width 0.25) (layer F.Cu) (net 17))
 (segment (start 192.84 98.78) (end 193.703599 97.916401) (width 0.25) (layer F.Cu) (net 17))
 (segment (start 196.494401 92.049599) (end 197.358 91.186) (width 0.25) (layer F.Cu) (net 18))
 (segment (start 193.655399 94.888601) (end 196.494401 92.049599) (width 0.25) (layer F.Cu) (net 18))
 (segment (start 191.651399 94.888601) (end 193.655399 94.888601) (width 0.25) (layer F.Cu) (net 18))
 (segment (start 190.3 96.24) (end 191.651399 94.888601) (width 0.25) (layer F.Cu) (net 18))
 (segment (start 199.034401 92.049599) (end 199.898 91.186) (width 0.25) (layer F.Cu) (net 19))
 (segment (start 198.709399 92.374601) (end 199.034401 92.049599) (width 0.25) (layer F.Cu) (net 19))
 (segment (start 196.950269 92.374601) (end 198.709399 92.374601) (width 0.25) (layer F.Cu) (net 19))
 (segment (start 193.948469 95.376401) (end 196.950269 92.374601) (width 0.25) (layer F.Cu) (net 19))
 (segment (start 193.703599 95.376401) (end 193.948469 95.376401) (width 0.25) (layer F.Cu) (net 19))
 (segment (start 192.84 96.24) (end 193.703599 95.376401) (width 0.25) (layer F.Cu) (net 19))
 (segment (start 196.494401 89.509599) (end 197.358 88.646) (width 0.25) (layer F.Cu) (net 20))
 (segment (start 193.655399 92.348601) (end 196.494401 89.509599) (width 0.25) (layer F.Cu) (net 20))
 (segment (start 191.651399 92.348601) (end 193.655399 92.348601) (width 0.25) (layer F.Cu) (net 20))
 (segment (start 190.3 93.7) (end 191.651399 92.348601) (width 0.25) (layer F.Cu) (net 20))
 (segment (start 199.034401 89.509599) (end 199.898 88.646) (width 0.25) (layer F.Cu) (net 21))
 (segment (start 198.709399 89.834601) (end 199.034401 89.509599) (width 0.25) (layer F.Cu) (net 21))
 (segment (start 196.950269 89.834601) (end 198.709399 89.834601) (width 0.25) (layer F.Cu) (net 21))
 (segment (start 193.948469 92.836401) (end 196.950269 89.834601) (width 0.25) (layer F.Cu) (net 21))
 (segment (start 193.703599 92.836401) (end 193.948469 92.836401) (width 0.25) (layer F.Cu) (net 21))
 (segment (start 192.84 93.7) (end 193.703599 92.836401) (width 0.25) (layer F.Cu) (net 21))
 (segment (start 196.494401 86.969599) (end 197.358 86.106) (width 0.25) (layer F.Cu) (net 22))
 (segment (start 193.655399 89.808601) (end 196.494401 86.969599) (width 0.25) (layer F.Cu) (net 22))
 (segment (start 191.651399 89.808601) (end 193.655399 89.808601) (width 0.25) (layer F.Cu) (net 22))
 (segment (start 190.3 91.16) (end 191.651399 89.808601) (width 0.25) (layer F.Cu) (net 22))
 (segment (start 199.034401 86.969599) (end 199.898 86.106) (width 0.25) (layer F.Cu) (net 23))
 (segment (start 198.709399 87.294601) (end 199.034401 86.969599) (width 0.25) (layer F.Cu) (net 23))
 (segment (start 196.950269 87.294601) (end 198.709399 87.294601) (width 0.25) (layer F.Cu) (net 23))
 (segment (start 193.948469 90.296401) (end 196.950269 87.294601) (width 0.25) (layer F.Cu) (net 23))
 (segment (start 193.703599 90.296401) (end 193.948469 90.296401) (width 0.25) (layer F.Cu) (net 23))
 (segment (start 192.84 91.16) (end 193.703599 90.296401) (width 0.25) (layer F.Cu) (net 23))
 (segment (start 196.494401 84.429599) (end 197.358 83.566) (width 0.25) (layer F.Cu) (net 24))
 (segment (start 193.655399 87.268601) (end 196.494401 84.429599) (width 0.25) (layer F.Cu) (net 24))
 (segment (start 191.651399 87.268601) (end 193.655399 87.268601) (width 0.25) (layer F.Cu) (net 24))
 (segment (start 190.3 88.62) (end 191.651399 87.268601) (width 0.25) (layer F.Cu) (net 24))
 (segment (start 199.034401 84.429599) (end 199.898 83.566) (width 0.25) (layer F.Cu) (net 25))
 (segment (start 198.546601 84.917399) (end 199.034401 84.429599) (width 0.25) (layer F.Cu) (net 25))
 (segment (start 196.787471 84.917399) (end 198.546601 84.917399) (width 0.25) (layer F.Cu) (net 25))
 (segment (start 193.948469 87.756401) (end 196.787471 84.917399) (width 0.25) (layer F.Cu) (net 25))
 (segment (start 193.703599 87.756401) (end 193.948469 87.756401) (width 0.25) (layer F.Cu) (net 25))
 (segment (start 192.84 88.62) (end 193.703599 87.756401) (width 0.25) (layer F.Cu) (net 25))
 (segment (start 196.494401 81.889599) (end 197.358 81.026) (width 0.25) (layer F.Cu) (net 26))
 (segment (start 193.655399 84.728601) (end 196.494401 81.889599) (width 0.25) (layer F.Cu) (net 26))
 (segment (start 191.651399 84.728601) (end 193.655399 84.728601) (width 0.25) (layer F.Cu) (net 26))
 (segment (start 190.3 86.08) (end 191.651399 84.728601) (width 0.25) (layer F.Cu) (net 26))
 (segment (start 199.034401 81.889599) (end 199.898 81.026) (width 0.25) (layer F.Cu) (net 27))
 (segment (start 198.709399 82.214601) (end 199.034401 81.889599) (width 0.25) (layer F.Cu) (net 27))
 (segment (start 196.950269 82.214601) (end 198.709399 82.214601) (width 0.25) (layer F.Cu) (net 27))
 (segment (start 193.948469 85.216401) (end 196.950269 82.214601) (width 0.25) (layer F.Cu) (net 27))
 (segment (start 193.703599 85.216401) (end 193.948469 85.216401) (width 0.25) (layer F.Cu) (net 27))
 (segment (start 192.84 86.08) (end 193.703599 85.216401) (width 0.25) (layer F.Cu) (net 27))
 (segment (start 196.494401 79.349599) (end 197.358 78.486) (width 0.25) (layer F.Cu) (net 28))
 (segment (start 193.655399 82.188601) (end 196.494401 79.349599) (width 0.25) (layer F.Cu) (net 28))
 (segment (start 191.651399 82.188601) (end 193.655399 82.188601) (width 0.25) (layer F.Cu) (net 28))
 (segment (start 190.3 83.54) (end 191.651399 82.188601) (width 0.25) (layer F.Cu) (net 28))
 (segment (start 199.034401 79.349599) (end 199.898 78.486) (width 0.25) (layer F.Cu) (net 29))
 (segment (start 198.709399 79.674601) (end 199.034401 79.349599) (width 0.25) (layer F.Cu) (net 29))
 (segment (start 196.950269 79.674601) (end 198.709399 79.674601) (width 0.25) (layer F.Cu) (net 29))
 (segment (start 193.948469 82.676401) (end 196.950269 79.674601) (width 0.25) (layer F.Cu) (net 29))
 (segment (start 193.703599 82.676401) (end 193.948469 82.676401) (width 0.25) (layer F.Cu) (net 29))
 (segment (start 192.84 83.54) (end 193.703599 82.676401) (width 0.25) (layer F.Cu) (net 29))
 (segment (start 196.494401 76.809599) (end 197.358 75.946) (width 0.25) (layer F.Cu) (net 30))
 (segment (start 193.655399 79.648601) (end 196.494401 76.809599) (width 0.25) (layer F.Cu) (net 30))
 (segment (start 191.651399 79.648601) (end 193.655399 79.648601) (width 0.25) (layer F.Cu) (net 30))
 (segment (start 190.3 81) (end 191.651399 79.648601) (width 0.25) (layer F.Cu) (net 30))
 (segment (start 199.034401 76.809599) (end 199.898 75.946) (width 0.25) (layer F.Cu) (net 31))
 (segment (start 198.709399 77.134601) (end 199.034401 76.809599) (width 0.25) (layer F.Cu) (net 31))
 (segment (start 196.950269 77.134601) (end 198.709399 77.134601) (width 0.25) (layer F.Cu) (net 31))
 (segment (start 193.948469 80.136401) (end 196.950269 77.134601) (width 0.25) (layer F.Cu) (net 31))
 (segment (start 193.703599 80.136401) (end 193.948469 80.136401) (width 0.25) (layer F.Cu) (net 31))
 (segment (start 192.84 81) (end 193.703599 80.136401) (width 0.25) (layer F.Cu) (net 31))
 (segment (start 196.494401 74.269599) (end 197.358 73.406) (width 0.25) (layer F.Cu) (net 32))
 (segment (start 193.492601 77.271399) (end 196.494401 74.269599) (width 0.25) (layer F.Cu) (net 32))
 (segment (start 191.488601 77.271399) (end 193.492601 77.271399) (width 0.25) (layer F.Cu) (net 32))
 (segment (start 190.3 78.46) (end 191.488601 77.271399) (width 0.25) (layer F.Cu) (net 32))
 (segment (start 199.034401 74.269599) (end 199.898 73.406) (width 0.25) (layer F.Cu) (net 33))
 (segment (start 198.709399 74.594601) (end 199.034401 74.269599) (width 0.25) (layer F.Cu) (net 33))
 (segment (start 196.950269 74.594601) (end 198.709399 74.594601) (width 0.25) (layer F.Cu) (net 33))
 (segment (start 193.08487 78.46) (end 196.950269 74.594601) (width 0.25) (layer F.Cu) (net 33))
 (segment (start 192.84 78.46) (end 193.08487 78.46) (width 0.25) (layer F.Cu) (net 33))
 (segment (start 197.358 71.142) (end 197.358 70.866) (width 1) (layer B.Cu) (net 34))
 (segment (start 192.84 75.384) (end 192.84 75.92) (width 0.25) (layer F.Cu) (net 34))
 (segment (start 189.078686 75.92) (end 190.3 75.92) (width 1.5) (layer B.Cu) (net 34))
 (segment (start 181.03 83.968686) (end 189.078686 75.92) (width 1.5) (layer B.Cu) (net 34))
 (segment (start 181.03 99.46) (end 181.03 83.968686) (width 1.5) (layer B.Cu) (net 34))
 (segment (start 192.84 75.92) (end 190.3 75.92) (width 1.5) (layer B.Cu) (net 34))
 (segment (start 199.898 70.866) (end 197.358 70.866) (width 1.5) (layer B.Cu) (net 34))
 (segment (start 192.84 74.698686) (end 192.84 75.92) (width 1.5) (layer B.Cu) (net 34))
 (segment (start 192.84 74.162686) (end 192.84 74.698686) (width 1.5) (layer B.Cu) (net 34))
 (segment (start 196.136686 70.866) (end 192.84 74.162686) (width 1.5) (layer B.Cu) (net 34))
 (segment (start 197.358 70.866) (end 196.136686 70.866) (width 1.5) (layer B.Cu) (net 34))
 (segment (start 182.3 100.780241) (end 182.3 102) (width 0.25) (layer F.Cu) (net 39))
 (segment (start 182.3 72.314) (end 182.3 100.780241) (width 0.25) (layer F.Cu) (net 39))
 (segment (start 182.118 72.132) (end 182.3 72.314) (width 0.25) (layer F.Cu) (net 39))
 (segment (start 182.118 70.866) (end 182.118 72.132) (width 0.25) (layer F.Cu) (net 39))
 (segment (start 184.658 98.372) (end 183.57 99.46) (width 0.25) (layer F.Cu) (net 40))
 (segment (start 184.658 70.866) (end 184.658 98.372) (width 0.25) (layer F.Cu) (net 40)))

